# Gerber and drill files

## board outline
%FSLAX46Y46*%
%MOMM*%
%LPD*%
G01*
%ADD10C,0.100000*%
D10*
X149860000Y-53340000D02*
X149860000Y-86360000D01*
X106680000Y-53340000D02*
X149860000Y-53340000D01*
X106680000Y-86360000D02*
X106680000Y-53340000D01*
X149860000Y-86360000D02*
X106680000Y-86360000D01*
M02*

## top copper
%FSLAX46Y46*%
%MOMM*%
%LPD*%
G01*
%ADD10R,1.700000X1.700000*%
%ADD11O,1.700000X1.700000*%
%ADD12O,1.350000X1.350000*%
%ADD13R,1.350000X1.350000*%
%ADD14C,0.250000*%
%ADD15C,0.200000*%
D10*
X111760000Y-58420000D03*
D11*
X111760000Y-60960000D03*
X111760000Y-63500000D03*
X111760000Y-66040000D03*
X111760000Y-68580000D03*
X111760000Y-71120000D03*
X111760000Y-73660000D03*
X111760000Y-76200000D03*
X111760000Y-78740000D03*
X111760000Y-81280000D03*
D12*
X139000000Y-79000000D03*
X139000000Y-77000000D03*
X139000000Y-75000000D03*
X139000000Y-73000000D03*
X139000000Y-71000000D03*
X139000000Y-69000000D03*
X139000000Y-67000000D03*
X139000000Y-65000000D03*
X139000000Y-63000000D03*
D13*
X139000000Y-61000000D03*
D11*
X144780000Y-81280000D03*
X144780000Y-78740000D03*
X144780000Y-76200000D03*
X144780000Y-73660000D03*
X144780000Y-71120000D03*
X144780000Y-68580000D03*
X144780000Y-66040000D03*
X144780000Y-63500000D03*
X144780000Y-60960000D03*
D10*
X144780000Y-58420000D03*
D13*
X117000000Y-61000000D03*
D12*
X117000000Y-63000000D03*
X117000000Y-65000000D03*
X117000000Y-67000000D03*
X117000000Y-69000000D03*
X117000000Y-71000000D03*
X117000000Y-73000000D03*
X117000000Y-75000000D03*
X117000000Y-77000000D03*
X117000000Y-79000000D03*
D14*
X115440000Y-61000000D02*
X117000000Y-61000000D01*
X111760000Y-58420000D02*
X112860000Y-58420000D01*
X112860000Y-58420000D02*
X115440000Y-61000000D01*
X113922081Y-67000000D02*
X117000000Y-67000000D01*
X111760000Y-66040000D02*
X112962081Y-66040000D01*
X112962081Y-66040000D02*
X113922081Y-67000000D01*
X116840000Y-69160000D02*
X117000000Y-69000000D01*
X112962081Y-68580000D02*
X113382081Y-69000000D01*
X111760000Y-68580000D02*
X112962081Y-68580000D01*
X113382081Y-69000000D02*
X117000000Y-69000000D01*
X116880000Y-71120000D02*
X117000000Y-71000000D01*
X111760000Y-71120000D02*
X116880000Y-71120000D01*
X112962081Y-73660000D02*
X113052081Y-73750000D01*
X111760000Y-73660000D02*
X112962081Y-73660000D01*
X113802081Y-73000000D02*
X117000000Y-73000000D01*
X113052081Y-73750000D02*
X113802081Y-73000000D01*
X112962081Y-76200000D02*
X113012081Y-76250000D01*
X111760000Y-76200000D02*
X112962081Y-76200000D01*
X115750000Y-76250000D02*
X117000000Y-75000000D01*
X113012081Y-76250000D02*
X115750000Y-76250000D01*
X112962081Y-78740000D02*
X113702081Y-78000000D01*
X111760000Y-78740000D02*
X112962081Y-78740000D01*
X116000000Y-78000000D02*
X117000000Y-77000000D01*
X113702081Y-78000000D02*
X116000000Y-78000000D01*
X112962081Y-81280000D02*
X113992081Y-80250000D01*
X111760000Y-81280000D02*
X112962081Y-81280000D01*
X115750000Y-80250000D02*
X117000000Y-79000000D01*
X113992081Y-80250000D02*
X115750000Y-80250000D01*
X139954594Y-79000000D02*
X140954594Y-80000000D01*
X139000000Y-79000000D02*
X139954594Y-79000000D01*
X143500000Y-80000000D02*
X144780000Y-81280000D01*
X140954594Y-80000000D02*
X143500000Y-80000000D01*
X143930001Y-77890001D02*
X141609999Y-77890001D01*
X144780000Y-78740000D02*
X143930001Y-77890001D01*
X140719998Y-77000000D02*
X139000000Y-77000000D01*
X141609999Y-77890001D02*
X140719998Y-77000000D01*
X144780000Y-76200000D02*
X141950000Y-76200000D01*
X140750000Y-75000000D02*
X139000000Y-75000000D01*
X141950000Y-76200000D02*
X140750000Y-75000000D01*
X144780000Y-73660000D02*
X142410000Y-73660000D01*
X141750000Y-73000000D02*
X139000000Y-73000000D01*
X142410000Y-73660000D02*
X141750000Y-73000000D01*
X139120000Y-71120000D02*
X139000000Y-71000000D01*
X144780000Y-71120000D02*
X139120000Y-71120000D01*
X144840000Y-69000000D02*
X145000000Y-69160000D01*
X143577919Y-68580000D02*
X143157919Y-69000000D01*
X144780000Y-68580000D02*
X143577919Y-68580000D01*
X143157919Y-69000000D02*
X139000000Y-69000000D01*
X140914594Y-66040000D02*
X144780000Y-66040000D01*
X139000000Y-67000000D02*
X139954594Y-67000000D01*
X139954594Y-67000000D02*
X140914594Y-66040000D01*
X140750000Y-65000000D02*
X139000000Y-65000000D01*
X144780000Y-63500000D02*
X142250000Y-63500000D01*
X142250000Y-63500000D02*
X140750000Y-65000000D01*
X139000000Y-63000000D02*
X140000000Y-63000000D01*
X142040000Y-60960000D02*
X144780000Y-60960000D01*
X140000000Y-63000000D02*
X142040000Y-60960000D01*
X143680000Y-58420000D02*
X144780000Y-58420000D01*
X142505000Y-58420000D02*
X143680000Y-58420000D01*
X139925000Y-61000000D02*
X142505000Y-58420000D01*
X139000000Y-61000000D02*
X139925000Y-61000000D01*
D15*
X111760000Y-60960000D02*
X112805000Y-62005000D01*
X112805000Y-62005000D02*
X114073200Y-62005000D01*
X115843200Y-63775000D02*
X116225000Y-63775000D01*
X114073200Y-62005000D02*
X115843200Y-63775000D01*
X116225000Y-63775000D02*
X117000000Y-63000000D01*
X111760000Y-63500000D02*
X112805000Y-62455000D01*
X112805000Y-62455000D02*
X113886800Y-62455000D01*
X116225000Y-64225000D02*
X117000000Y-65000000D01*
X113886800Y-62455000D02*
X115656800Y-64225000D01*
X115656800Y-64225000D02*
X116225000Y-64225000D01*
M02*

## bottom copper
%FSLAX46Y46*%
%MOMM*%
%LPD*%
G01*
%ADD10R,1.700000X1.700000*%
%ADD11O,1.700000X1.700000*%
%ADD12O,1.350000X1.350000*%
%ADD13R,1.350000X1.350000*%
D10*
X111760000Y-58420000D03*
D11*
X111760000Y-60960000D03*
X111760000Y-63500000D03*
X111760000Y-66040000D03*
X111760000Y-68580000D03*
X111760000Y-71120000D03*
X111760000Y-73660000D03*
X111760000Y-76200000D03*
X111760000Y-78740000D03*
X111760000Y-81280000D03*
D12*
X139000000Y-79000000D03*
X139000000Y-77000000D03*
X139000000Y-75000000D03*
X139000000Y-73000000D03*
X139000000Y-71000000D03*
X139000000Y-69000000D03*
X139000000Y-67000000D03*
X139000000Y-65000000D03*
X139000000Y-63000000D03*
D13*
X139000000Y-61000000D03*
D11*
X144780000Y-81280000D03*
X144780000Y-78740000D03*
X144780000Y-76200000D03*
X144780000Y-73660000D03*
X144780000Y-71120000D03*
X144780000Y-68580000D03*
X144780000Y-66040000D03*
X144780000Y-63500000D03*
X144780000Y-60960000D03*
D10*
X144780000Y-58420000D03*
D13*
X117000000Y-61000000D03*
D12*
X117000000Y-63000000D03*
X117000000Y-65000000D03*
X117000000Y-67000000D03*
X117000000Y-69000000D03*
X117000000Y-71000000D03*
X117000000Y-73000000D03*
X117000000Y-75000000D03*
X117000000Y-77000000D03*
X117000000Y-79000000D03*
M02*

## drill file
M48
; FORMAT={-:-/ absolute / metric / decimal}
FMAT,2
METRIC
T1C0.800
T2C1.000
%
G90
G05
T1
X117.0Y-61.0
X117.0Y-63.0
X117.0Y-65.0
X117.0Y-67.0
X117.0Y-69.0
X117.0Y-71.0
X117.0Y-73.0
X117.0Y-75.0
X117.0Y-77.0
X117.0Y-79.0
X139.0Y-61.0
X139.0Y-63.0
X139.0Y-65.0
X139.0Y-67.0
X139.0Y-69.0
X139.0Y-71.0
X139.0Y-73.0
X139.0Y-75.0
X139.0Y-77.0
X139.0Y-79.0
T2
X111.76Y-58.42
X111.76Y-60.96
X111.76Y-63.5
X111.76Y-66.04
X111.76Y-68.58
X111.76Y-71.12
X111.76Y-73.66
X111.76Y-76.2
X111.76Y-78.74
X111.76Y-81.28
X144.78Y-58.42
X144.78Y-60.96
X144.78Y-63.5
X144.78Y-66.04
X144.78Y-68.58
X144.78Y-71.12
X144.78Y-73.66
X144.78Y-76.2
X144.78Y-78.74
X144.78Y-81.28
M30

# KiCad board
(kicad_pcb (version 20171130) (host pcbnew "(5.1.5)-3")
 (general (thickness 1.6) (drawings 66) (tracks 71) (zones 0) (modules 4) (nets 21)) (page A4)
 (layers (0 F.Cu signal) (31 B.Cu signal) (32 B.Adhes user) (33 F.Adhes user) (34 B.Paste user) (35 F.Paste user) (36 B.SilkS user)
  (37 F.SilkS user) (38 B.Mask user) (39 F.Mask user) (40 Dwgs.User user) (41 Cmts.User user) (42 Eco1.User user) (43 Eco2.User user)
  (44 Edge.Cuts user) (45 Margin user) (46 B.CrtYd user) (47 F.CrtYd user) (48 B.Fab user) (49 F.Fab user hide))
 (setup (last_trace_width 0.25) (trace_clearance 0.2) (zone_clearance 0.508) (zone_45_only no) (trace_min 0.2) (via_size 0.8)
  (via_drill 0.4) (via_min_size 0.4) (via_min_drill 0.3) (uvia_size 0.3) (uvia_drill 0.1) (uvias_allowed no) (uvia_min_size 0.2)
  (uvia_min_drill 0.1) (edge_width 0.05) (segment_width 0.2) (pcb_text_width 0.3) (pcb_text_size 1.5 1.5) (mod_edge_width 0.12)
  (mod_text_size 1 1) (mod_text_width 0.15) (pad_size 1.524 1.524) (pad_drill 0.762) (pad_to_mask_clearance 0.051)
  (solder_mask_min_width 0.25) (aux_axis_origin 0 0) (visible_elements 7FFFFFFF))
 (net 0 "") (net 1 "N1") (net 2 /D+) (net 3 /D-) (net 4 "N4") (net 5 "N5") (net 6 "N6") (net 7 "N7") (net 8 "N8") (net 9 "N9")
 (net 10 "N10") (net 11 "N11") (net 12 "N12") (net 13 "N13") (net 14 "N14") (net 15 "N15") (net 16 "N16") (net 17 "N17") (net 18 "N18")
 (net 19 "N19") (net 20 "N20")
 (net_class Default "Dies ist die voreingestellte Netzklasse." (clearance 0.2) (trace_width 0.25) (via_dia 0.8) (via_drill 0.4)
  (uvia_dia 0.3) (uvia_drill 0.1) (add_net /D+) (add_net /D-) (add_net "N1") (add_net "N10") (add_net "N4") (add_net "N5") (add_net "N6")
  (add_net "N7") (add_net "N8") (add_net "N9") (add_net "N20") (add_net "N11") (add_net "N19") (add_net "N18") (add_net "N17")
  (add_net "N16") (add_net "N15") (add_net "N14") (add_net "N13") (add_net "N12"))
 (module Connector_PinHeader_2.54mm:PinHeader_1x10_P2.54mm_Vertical (layer F.Cu) (at 111.76 58.42)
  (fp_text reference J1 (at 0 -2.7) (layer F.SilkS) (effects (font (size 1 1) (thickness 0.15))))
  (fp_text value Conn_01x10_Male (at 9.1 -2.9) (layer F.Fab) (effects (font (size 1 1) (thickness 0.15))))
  (pad 1 thru_hole rect (at 0 0) (size 1.7 1.7) (drill 1) (layers *.Cu *.Mask) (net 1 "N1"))
  (pad 2 thru_hole oval (at 0 2.54) (size 1.7 1.7) (drill 1) (layers *.Cu *.Mask) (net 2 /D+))
  (pad 3 thru_hole oval (at 0 5.08) (size 1.7 1.7) (drill 1) (layers *.Cu *.Mask) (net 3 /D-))
  (pad 4 thru_hole oval (at 0 7.62) (size 1.7 1.7) (drill 1) (layers *.Cu *.Mask) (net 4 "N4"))
  (pad 5 thru_hole oval (at 0 10.16) (size 1.7 1.7) (drill 1) (layers *.Cu *.Mask) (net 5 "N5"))
  (pad 6 thru_hole oval (at 0 12.7) (size 1.7 1.7) (drill 1) (layers *.Cu *.Mask) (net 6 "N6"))
  (pad 7 thru_hole oval (at 0 15.24) (size 1.7 1.7) (drill 1) (layers *.Cu *.Mask) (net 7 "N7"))
  (pad 8 thru_hole oval (at 0 17.78) (size 1.7 1.7) (drill 1) (layers *.Cu *.Mask) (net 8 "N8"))
  (pad 9 thru_hole oval (at 0 20.32) (size 1.7 1.7) (drill 1) (layers *.Cu *.Mask) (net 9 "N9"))
  (pad 10 thru_hole oval (at 0 22.86) (size 1.7 1.7) (drill 1) (layers *.Cu *.Mask) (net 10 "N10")))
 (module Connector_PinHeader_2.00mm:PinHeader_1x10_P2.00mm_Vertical (layer F.Cu) (at 139 61)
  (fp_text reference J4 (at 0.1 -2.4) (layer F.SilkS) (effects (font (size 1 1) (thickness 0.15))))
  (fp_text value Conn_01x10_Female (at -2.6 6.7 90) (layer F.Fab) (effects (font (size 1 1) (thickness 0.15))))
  (pad 10 thru_hole oval (at 0 18) (size 1.35 1.35) (drill 0.8) (layers *.Cu *.Mask) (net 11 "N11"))
  (pad 9 thru_hole oval (at 0 16) (size 1.35 1.35) (drill 0.8) (layers *.Cu *.Mask) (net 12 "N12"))
  (pad 8 thru_hole oval (at 0 14) (size 1.35 1.35) (drill 0.8) (layers *.Cu *.Mask) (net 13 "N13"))
  (pad 7 thru_hole oval (at 0 12) (size 1.35 1.35) (drill 0.8) (layers *.Cu *.Mask) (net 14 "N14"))
  (pad 6 thru_hole oval (at 0 10) (size 1.35 1.35) (drill 0.8) (layers *.Cu *.Mask) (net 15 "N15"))
  (pad 5 thru_hole oval (at 0 8) (size 1.35 1.35) (drill 0.8) (layers *.Cu *.Mask) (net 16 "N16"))
  (pad 4 thru_hole oval (at 0 6) (size 1.35 1.35) (drill 0.8) (layers *.Cu *.Mask) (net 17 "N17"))
  (pad 3 thru_hole oval (at 0 4) (size 1.35 1.35) (drill 0.8) (layers *.Cu *.Mask) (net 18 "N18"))
  (pad 2 thru_hole oval (at 0 2) (size 1.35 1.35) (drill 0.8) (layers *.Cu *.Mask) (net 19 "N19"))
  (pad 1 thru_hole rect (at 0 0) (size 1.35 1.35) (drill 0.8) (layers *.Cu *.Mask) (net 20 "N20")))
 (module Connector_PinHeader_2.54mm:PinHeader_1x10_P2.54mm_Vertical (layer F.Cu) (at 144.78 58.42)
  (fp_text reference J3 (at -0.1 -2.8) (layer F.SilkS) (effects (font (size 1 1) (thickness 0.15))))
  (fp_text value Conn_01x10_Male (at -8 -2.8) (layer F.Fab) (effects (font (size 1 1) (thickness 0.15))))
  (pad 10 thru_hole oval (at 0 22.86) (size 1.7 1.7) (drill 1) (layers *.Cu *.Mask) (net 11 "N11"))
  (pad 9 thru_hole oval (at 0 20.32) (size 1.7 1.7) (drill 1) (layers *.Cu *.Mask) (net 12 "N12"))
  (pad 8 thru_hole oval (at 0 17.78) (size 1.7 1.7) (drill 1) (layers *.Cu *.Mask) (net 13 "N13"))
  (pad 7 thru_hole oval (at 0 15.24) (size 1.7 1.7) (drill 1) (layers *.Cu *.Mask) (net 14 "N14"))
  (pad 6 thru_hole oval (at 0 12.7) (size 1.7 1.7) (drill 1) (layers *.Cu *.Mask) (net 15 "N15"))
  (pad 5 thru_hole oval (at 0 10.16) (size 1.7 1.7) (drill 1) (layers *.Cu *.Mask) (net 16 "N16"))
  (pad 4 thru_hole oval (at 0 7.62) (size 1.7 1.7) (drill 1) (layers *.Cu *.Mask) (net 17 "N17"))
  (pad 3 thru_hole oval (at 0 5.08) (size 1.7 1.7) (drill 1) (layers *.Cu *.Mask) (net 18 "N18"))
  (pad 2 thru_hole oval (at 0 2.54) (size 1.7 1.7) (drill 1) (layers *.Cu *.Mask) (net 19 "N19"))
  (pad 1 thru_hole rect (at 0 0) (size 1.7 1.7) (drill 1) (layers *.Cu *.Mask) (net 20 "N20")))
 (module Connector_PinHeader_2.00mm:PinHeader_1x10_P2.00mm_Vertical (layer F.Cu) (at 117 61)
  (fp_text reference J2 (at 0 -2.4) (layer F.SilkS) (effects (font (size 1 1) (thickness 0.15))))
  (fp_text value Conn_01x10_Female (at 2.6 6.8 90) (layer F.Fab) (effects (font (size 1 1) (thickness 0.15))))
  (pad 1 thru_hole rect (at 0 0) (size 1.35 1.35) (drill 0.8) (layers *.Cu *.Mask) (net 1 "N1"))
  (pad 2 thru_hole oval (at 0 2) (size 1.35 1.35) (drill 0.8) (layers *.Cu *.Mask) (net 2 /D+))
  (pad 3 thru_hole oval (at 0 4) (size 1.35 1.35) (drill 0.8) (layers *.Cu *.Mask) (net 3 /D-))
  (pad 4 thru_hole oval (at 0 6) (size 1.35 1.35) (drill 0.8) (layers *.Cu *.Mask) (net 4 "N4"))
  (pad 5 thru_hole oval (at 0 8) (size 1.35 1.35) (drill 0.8) (layers *.Cu *.Mask) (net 5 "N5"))
  (pad 6 thru_hole oval (at 0 10) (size 1.35 1.35) (drill 0.8) (layers *.Cu *.Mask) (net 6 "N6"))
  (pad 7 thru_hole oval (at 0 12) (size 1.35 1.35) (drill 0.8) (layers *.Cu *.Mask) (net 7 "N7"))
  (pad 8 thru_hole oval (at 0 14) (size 1.35 1.35) (drill 0.8) (layers *.Cu *.Mask) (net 8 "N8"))
  (pad 9 thru_hole oval (at 0 16) (size 1.35 1.35) (drill 0.8) (layers *.Cu *.Mask) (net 9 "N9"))
  (pad 10 thru_hole oval (at 0 18) (size 1.35 1.35) (drill 0.8) (layers *.Cu *.Mask) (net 10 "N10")))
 (gr_line (start 149.86 53.34) (end 149.86 86.36) (layer Edge.Cuts) (width 0.1))
 (gr_line (start 106.68 53.34) (end 149.86 53.34) (layer Edge.Cuts) (width 0.1))
 (gr_line (start 106.68 86.36) (end 106.68 53.34) (layer Edge.Cuts) (width 0.1))
 (gr_line (start 149.86 86.36) (end 106.68 86.36) (layer Edge.Cuts) (width 0.1))
 (segment (start 115.44 61) (end 117 61) (width 0.25) (layer F.Cu) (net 1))
 (segment (start 111.76 58.42) (end 112.86 58.42) (width 0.25) (layer F.Cu) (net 1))
 (segment (start 112.86 58.42) (end 115.44 61) (width 0.25) (layer F.Cu) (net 1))
 (segment (start 113.922081 67) (end 117 67) (width 0.25) (layer F.Cu) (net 4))
 (segment (start 111.76 66.04) (end 112.962081 66.04) (width 0.25) (layer F.Cu) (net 4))
 (segment (start 112.962081 66.04) (end 113.922081 67) (width 0.25) (layer F.Cu) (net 4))
 (segment (start 116.84 69.16) (end 117 69) (width 0.25) (layer F.Cu) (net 5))
 (segment (start 112.962081 68.58) (end 113.382081 69) (width 0.25) (layer F.Cu) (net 5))
 (segment (start 111.76 68.58) (end 112.962081 68.58) (width 0.25) (layer F.Cu) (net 5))
 (segment (start 113.382081 69) (end 117 69) (width 0.25) (layer F.Cu) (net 5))
 (segment (start 116.88 71.12) (end 117 71) (width 0.25) (layer F.Cu) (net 6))
 (segment (start 111.76 71.12) (end 116.88 71.12) (width 0.25) (layer F.Cu) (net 6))
 (segment (start 112.962081 73.66) (end 113.052081 73.75) (width 0.25) (layer F.Cu) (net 7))
 (segment (start 111.76 73.66) (end 112.962081 73.66) (width 0.25) (layer F.Cu) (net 7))
 (segment (start 113.802081 73) (end 117 73) (width 0.25) (layer F.Cu) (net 7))
 (segment (start 113.052081 73.75) (end 113.802081 73) (width 0.25) (layer F.Cu) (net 7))
 (segment (start 112.962081 76.2) (end 113.012081 76.25) (width 0.25) (layer F.Cu) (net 8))
 (segment (start 111.76 76.2) (end 112.962081 76.2) (width 0.25) (layer F.Cu) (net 8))
 (segment (start 115.75 76.25) (end 117 75) (width 0.25) (layer F.Cu) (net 8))
 (segment (start 113.012081 76.25) (end 115.75 76.25) (width 0.25) (layer F.Cu) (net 8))
 (segment (start 112.962081 78.74) (end 113.702081 78) (width 0.25) (layer F.Cu) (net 9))
 (segment (start 111.76 78.74) (end 112.962081 78.74) (width 0.25) (layer F.Cu) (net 9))
 (segment (start 116 78) (end 117 77) (width 0.25) (layer F.Cu) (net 9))
 (segment (start 113.702081 78) (end 116 78) (width 0.25) (layer F.Cu) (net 9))
 (segment (start 112.962081 81.28) (end 113.992081 80.25) (width 0.25) (layer F.Cu) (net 10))
 (segment (start 111.76 81.28) (end 112.962081 81.28) (width 0.25) (layer F.Cu) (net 10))
 (segment (start 115.75 80.25) (end 117 79) (width 0.25) (layer F.Cu) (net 10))
 (segment (start 113.992081 80.25) (end 115.75 80.25) (width 0.25) (layer F.Cu) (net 10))
 (segment (start 139.954594 79) (end 140.954594 80) (width 0.25) (layer F.Cu) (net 11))
 (segment (start 139 79) (end 139.954594 79) (width 0.25) (layer F.Cu) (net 11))
 (segment (start 143.5 80) (end 144.78 81.28) (width 0.25) (layer F.Cu) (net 11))
 (segment (start 140.954594 80) (end 143.5 80) (width 0.25) (layer F.Cu) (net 11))
 (segment (start 143.930001 77.890001) (end 141.609999 77.890001) (width 0.25) (layer F.Cu) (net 12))
 (segment (start 144.78 78.74) (end 143.930001 77.890001) (width 0.25) (layer F.Cu) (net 12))
 (segment (start 140.719998 77) (end 139 77) (width 0.25) (layer F.Cu) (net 12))
 (segment (start 141.609999 77.890001) (end 140.719998 77) (width 0.25) (layer F.Cu) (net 12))
 (segment (start 144.78 76.2) (end 141.95 76.2) (width 0.25) (layer F.Cu) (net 13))
 (segment (start 140.75 75) (end 139 75) (width 0.25) (layer F.Cu) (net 13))
 (segment (start 141.95 76.2) (end 140.75 75) (width 0.25) (layer F.Cu) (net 13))
 (segment (start 144.78 73.66) (end 142.41 73.66) (width 0.25) (layer F.Cu) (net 14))
 (segment (start 141.75 73) (end 139 73) (width 0.25) (layer F.Cu) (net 14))
 (segment (start 142.41 73.66) (end 141.75 73) (width 0.25) (layer F.Cu) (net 14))
 (segment (start 139.12 71.12) (end 139 71) (width 0.25) (layer F.Cu) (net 15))
 (segment (start 144.78 71.12) (end 139.12 71.12) (width 0.25) (layer F.Cu) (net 15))
 (segment (start 144.84 69) (end 145 69.16) (width 0.25) (layer F.Cu) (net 16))
 (segment (start 143.577919 68.58) (end 143.157919 69) (width 0.25) (layer F.Cu) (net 16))
 (segment (start 144.78 68.58) (end 143.577919 68.58) (width 0.25) (layer F.Cu) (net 16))
 (segment (start 143.157919 69) (end 139 69) (width 0.25) (layer F.Cu) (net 16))
 (segment (start 140.914594 66.04) (end 144.78 66.04) (width 0.25) (layer F.Cu) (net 17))
 (segment (start 139 67) (end 139.954594 67) (width 0.25) (layer F.Cu) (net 17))
 (segment (start 139.954594 67) (end 140.914594 66.04) (width 0.25) (layer F.Cu) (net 17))
 (segment (start 140.75 65) (end 139 65) (width 0.25) (layer F.Cu) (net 18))
 (segment (start 144.78 63.5) (end 142.25 63.5) (width 0.25) (layer F.Cu) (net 18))
 (segment (start 142.25 63.5) (end 140.75 65) (width 0.25) (layer F.Cu) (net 18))
 (segment (start 139 63) (end 140 63) (width 0.25) (layer F.Cu) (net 19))
 (segment (start 142.04 60.96) (end 144.78 60.96) (width 0.25) (layer F.Cu) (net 19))
 (segment (start 140 63) (end 142.04 60.96) (width 0.25) (layer F.Cu) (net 19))
 (segment (start 143.68 58.42) (end 144.78 58.42) (width 0.25) (layer F.Cu) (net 20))
 (segment (start 142.505 58.42) (end 143.68 58.42) (width 0.25) (layer F.Cu) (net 20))
 (segment (start 139.925 61) (end 142.505 58.42) (width 0.25) (layer F.Cu) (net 20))
 (segment (start 139 61) (end 139.925 61) (width 0.25) (layer F.Cu) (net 20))
 (segment (start 111.76 60.96) (end 112.805 62.005) (width 0.2) (layer F.Cu) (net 2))
 (segment (start 112.805 62.005) (end 114.0732 62.005) (width 0.2) (layer F.Cu) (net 2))
 (segment (start 115.8432 63.775) (end 116.225 63.775) (width 0.2) (layer F.Cu) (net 2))
 (segment (start 114.0732 62.005) (end 115.8432 63.775) (width 0.2) (layer F.Cu) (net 2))
 (segment (start 116.225 63.775) (end 117 63) (width 0.2) (layer F.Cu) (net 2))
 (segment (start 111.76 63.5) (end 112.805 62.455) (width 0.2) (layer F.Cu) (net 3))
 (segment (start 112.805 62.455) (end 113.8868 62.455) (width 0.2) (layer F.Cu) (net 3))
 (segment (start 116.225 64.225) (end 117 65) (width 0.2) (layer F.Cu) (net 3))
 (segment (start 113.8868 62.455) (end 115.6568 64.225) (width 0.2) (layer F.Cu) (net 3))
 (segment (start 115.6568 64.225) (end 116.225 64.225) (width 0.2) (layer F.Cu) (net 3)))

